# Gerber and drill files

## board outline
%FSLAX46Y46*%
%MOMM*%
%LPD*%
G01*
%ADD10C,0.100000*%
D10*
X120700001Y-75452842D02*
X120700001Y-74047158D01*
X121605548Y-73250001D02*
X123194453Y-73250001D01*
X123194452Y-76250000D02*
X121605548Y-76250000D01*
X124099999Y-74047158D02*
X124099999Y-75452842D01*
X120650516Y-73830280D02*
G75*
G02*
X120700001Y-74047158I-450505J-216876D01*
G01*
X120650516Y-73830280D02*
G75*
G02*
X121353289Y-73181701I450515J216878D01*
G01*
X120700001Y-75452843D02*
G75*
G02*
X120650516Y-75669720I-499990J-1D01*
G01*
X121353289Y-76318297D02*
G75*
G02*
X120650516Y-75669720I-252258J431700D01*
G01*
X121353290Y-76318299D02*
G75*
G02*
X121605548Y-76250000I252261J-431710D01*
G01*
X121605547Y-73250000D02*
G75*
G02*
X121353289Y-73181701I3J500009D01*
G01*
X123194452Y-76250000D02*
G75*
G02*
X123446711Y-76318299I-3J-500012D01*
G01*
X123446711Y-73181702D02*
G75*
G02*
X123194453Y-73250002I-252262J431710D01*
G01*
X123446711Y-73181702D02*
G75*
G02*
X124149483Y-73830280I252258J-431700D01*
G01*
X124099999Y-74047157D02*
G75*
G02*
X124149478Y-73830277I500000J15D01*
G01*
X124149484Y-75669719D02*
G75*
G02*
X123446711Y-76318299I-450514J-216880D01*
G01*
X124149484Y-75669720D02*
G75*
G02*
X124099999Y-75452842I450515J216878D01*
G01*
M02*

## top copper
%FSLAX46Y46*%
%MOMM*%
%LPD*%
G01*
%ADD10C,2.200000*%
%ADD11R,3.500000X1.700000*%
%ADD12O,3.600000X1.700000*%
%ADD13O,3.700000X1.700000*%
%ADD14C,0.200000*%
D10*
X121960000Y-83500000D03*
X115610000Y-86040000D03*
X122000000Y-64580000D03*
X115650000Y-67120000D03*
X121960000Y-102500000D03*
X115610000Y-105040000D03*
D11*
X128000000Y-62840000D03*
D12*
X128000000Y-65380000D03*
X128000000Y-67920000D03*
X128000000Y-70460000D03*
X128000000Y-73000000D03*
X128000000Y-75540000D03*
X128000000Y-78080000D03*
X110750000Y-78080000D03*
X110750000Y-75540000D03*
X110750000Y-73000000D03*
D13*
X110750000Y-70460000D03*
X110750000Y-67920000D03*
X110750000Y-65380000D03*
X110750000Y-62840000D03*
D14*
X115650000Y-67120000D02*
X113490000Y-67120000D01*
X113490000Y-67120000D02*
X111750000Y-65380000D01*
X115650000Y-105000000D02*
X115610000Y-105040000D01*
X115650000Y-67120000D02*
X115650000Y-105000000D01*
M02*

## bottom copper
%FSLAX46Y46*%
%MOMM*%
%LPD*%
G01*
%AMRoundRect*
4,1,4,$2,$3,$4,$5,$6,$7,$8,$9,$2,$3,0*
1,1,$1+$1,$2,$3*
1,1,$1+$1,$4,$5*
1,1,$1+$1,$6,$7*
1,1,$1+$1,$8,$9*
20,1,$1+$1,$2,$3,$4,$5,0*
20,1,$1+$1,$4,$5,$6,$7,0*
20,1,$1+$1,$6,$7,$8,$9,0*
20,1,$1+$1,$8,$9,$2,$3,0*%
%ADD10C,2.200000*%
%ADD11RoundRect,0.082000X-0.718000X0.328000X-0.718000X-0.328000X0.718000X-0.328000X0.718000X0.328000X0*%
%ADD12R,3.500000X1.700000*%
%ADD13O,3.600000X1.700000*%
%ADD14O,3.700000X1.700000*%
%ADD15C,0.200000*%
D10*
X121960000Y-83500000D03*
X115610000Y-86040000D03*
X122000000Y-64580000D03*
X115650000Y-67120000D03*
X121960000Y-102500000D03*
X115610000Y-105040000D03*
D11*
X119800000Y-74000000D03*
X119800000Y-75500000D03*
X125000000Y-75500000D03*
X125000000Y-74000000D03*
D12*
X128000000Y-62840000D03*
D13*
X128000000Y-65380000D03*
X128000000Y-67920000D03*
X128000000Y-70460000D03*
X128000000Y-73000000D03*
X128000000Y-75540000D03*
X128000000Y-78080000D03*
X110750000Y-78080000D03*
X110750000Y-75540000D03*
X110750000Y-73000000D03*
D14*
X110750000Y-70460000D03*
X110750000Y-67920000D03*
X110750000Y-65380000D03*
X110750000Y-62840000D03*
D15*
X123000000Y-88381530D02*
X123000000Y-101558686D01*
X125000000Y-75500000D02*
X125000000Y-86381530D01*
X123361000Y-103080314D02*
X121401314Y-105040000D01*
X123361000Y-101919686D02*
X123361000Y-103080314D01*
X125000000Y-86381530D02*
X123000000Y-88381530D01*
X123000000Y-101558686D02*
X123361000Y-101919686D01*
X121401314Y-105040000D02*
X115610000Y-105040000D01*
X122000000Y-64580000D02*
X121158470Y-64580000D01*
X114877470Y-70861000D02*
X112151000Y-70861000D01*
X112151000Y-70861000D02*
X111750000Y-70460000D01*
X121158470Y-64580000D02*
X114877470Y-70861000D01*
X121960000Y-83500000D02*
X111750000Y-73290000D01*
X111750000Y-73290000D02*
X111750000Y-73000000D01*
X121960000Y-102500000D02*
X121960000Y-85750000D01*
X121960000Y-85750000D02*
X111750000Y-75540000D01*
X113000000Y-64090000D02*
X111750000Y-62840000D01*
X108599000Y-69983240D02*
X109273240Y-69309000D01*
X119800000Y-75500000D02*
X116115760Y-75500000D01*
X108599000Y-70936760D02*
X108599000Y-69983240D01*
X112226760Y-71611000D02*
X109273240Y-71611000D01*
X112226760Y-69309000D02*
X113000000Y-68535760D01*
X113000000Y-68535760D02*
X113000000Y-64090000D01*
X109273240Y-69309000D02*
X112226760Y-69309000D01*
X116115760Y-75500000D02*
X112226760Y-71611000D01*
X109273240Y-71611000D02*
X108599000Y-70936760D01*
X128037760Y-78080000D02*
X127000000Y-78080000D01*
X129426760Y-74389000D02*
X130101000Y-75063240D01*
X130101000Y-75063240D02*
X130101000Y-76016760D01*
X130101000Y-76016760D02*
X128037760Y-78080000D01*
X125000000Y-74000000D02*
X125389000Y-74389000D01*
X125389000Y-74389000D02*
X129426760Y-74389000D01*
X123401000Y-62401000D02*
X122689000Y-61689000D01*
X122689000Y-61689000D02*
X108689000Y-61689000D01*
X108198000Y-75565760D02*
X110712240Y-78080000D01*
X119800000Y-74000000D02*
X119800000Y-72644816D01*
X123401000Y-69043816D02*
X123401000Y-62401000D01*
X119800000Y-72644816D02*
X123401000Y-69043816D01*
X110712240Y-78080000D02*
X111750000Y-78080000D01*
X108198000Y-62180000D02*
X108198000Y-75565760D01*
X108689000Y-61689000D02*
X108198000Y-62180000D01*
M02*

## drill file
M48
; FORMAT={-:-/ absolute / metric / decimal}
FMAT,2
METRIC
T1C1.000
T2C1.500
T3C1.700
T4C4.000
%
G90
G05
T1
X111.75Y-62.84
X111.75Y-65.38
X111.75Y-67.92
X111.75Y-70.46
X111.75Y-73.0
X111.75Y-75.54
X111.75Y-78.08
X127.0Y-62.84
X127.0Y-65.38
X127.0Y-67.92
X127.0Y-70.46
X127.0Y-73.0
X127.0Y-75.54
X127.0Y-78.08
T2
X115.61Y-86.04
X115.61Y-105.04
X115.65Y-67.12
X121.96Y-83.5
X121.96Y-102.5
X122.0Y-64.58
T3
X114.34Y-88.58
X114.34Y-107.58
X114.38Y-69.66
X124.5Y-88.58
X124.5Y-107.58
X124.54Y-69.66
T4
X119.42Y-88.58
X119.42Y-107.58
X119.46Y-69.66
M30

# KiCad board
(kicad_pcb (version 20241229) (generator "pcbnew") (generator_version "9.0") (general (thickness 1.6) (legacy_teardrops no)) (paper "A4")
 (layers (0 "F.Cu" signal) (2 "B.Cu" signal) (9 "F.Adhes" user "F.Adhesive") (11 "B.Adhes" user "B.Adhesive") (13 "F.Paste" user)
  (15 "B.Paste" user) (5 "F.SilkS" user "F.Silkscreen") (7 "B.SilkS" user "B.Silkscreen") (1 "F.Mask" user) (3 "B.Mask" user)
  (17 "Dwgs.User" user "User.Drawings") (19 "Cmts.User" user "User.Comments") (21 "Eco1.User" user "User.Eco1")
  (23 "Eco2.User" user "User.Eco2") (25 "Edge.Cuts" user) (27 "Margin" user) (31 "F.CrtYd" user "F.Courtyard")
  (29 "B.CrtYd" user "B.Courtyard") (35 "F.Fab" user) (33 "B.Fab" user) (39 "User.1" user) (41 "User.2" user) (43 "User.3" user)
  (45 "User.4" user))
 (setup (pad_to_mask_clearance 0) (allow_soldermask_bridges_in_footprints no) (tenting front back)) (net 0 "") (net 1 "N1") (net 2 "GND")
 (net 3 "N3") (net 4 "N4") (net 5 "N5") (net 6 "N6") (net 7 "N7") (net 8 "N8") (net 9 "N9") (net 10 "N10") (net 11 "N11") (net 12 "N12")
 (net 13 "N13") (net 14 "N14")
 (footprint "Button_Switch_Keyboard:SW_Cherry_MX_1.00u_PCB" (layer "F.Cu") (at 121.96 83.5)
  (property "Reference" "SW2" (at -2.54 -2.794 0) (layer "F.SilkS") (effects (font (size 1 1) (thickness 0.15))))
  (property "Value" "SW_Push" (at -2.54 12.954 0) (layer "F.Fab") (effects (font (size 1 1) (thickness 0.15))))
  (pad "" np_thru_hole circle (at -7.62 5.08) (size 1.7 1.7) (drill 1.7) (layers "*.Cu" "*.Mask"))
  (pad "" np_thru_hole circle (at -2.54 5.08) (size 4 4) (drill 4) (layers "*.Cu" "*.Mask"))
  (pad "" np_thru_hole circle (at 2.54 5.08) (size 1.7 1.7) (drill 1.7) (layers "*.Cu" "*.Mask"))
  (pad "1" thru_hole circle (at 0 0) (size 2.2 2.2) (drill 1.5) (layers "*.Cu" "*.Mask") (remove_unused_layers no) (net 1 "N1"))
  (pad "2" thru_hole circle (at -6.35 2.54) (size 2.2 2.2) (drill 1.5) (layers "*.Cu" "*.Mask") (remove_unused_layers no) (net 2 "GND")))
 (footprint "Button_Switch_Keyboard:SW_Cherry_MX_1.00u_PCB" (layer "F.Cu") (at 122 64.58)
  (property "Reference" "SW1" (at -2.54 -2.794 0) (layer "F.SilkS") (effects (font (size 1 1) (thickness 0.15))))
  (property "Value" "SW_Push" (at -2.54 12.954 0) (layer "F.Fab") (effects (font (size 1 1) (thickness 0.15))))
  (pad "" np_thru_hole circle (at -7.62 5.08) (size 1.7 1.7) (drill 1.7) (layers "*.Cu" "*.Mask"))
  (pad "" np_thru_hole circle (at -2.54 5.08) (size 4 4) (drill 4) (layers "*.Cu" "*.Mask"))
  (pad "" np_thru_hole circle (at 2.54 5.08) (size 1.7 1.7) (drill 1.7) (layers "*.Cu" "*.Mask"))
  (pad "1" thru_hole circle (at 0 0) (size 2.2 2.2) (drill 1.5) (layers "*.Cu" "*.Mask") (remove_unused_layers no) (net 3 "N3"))
  (pad "2" thru_hole circle (at -6.35 2.54) (size 2.2 2.2) (drill 1.5) (layers "*.Cu" "*.Mask") (remove_unused_layers no) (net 2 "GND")))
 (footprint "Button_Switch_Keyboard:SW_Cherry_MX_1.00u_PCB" (layer "F.Cu") (at 121.96 102.5)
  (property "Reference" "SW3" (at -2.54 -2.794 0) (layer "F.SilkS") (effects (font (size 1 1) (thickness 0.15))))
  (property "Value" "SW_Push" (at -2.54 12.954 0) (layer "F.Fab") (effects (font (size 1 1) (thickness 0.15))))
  (pad "" np_thru_hole circle (at -7.62 5.08) (size 1.7 1.7) (drill 1.7) (layers "*.Cu" "*.Mask"))
  (pad "" np_thru_hole circle (at -2.54 5.08) (size 4 4) (drill 4) (layers "*.Cu" "*.Mask"))
  (pad "" np_thru_hole circle (at 2.54 5.08) (size 1.7 1.7) (drill 1.7) (layers "*.Cu" "*.Mask"))
  (pad "1" thru_hole circle (at 0 0) (size 2.2 2.2) (drill 1.5) (layers "*.Cu" "*.Mask") (remove_unused_layers no) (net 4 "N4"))
  (pad "2" thru_hole circle (at -6.35 2.54) (size 2.2 2.2) (drill 1.5) (layers "*.Cu" "*.Mask") (remove_unused_layers no) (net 2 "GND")))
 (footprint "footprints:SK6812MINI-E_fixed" (layer "F.Cu") (at 122.399999 74.852842)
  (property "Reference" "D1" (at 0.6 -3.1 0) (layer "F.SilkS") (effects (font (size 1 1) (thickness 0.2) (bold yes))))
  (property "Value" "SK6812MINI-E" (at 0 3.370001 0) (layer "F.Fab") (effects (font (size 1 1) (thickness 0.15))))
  (fp_line (start -1.699998 0.6) (end -1.699998 -0.805684) (stroke (width 0.1) (type solid)) (layer "Edge.Cuts"))
  (fp_line (start -0.794451 -1.602841) (end 0.794454 -1.602841) (stroke (width 0.1) (type solid)) (layer "Edge.Cuts"))
  (fp_line (start 0.794453 1.397158) (end -0.794451 1.397158) (stroke (width 0.1) (type solid)) (layer "Edge.Cuts"))
  (fp_line (start 1.7 -0.805684) (end 1.7 0.6) (stroke (width 0.1) (type solid)) (layer "Edge.Cuts"))
  (fp_arc (start -1.749483 -1.022562) (mid -1.712526 -0.91691) (end -1.699998 -0.805684) (stroke (width 0.1) (type solid))
   (layer "Edge.Cuts"))
  (fp_arc (start -1.749483 -1.022562) (mid -1.63807 -1.606877) (end -1.04671 -1.671141) (stroke (width 0.1) (type solid))
   (layer "Edge.Cuts"))
  (fp_arc (start -1.699998 0.600001) (mid -1.712526 0.711226) (end -1.749483 0.816878) (stroke (width 0.1) (type solid)) (layer "Edge.Cuts"))
  (fp_arc (start -1.04671 1.465455) (mid -1.638069 1.401192) (end -1.749483 0.816878) (stroke (width 0.1) (type solid)) (layer "Edge.Cuts"))
  (fp_arc (start -1.046709 1.465457) (mid -0.925121 1.414535) (end -0.794451 1.397158) (stroke (width 0.1) (type solid)) (layer "Edge.Cuts"))
  (fp_arc (start -0.794452 -1.602842) (mid -0.925122 -1.620219) (end -1.04671 -1.671141) (stroke (width 0.1) (type solid))
   (layer "Edge.Cuts"))
  (fp_arc (start 0.794453 1.397158) (mid 0.925124 1.414535) (end 1.046712 1.465457) (stroke (width 0.1) (type solid)) (layer "Edge.Cuts"))
  (fp_arc (start 1.046712 -1.67114) (mid 0.925124 -1.620218) (end 0.794454 -1.602841) (stroke (width 0.1) (type solid)) (layer "Edge.Cuts"))
  (fp_arc (start 1.046712 -1.67114) (mid 1.638072 -1.606876) (end 1.749485 -1.022562) (stroke (width 0.1) (type solid)) (layer "Edge.Cuts"))
  (fp_arc (start 1.7 -0.805685) (mid 1.712528 -0.91691) (end 1.749485 -1.022562) (stroke (width 0.1) (type solid)) (layer "Edge.Cuts"))
  (fp_arc (start 1.749485 0.816877) (mid 1.638073 1.401193) (end 1.046712 1.465457) (stroke (width 0.1) (type solid)) (layer "Edge.Cuts"))
  (fp_arc (start 1.749485 0.816878) (mid 1.712528 0.711226) (end 1.7 0.6) (stroke (width 0.1) (type solid)) (layer "Edge.Cuts"))
  (pad "1" smd roundrect (at -2.599999 -0.852842 270) (size 0.82 1.6) (layers "B.Cu" "B.Mask" "B.Paste") (roundrect_rratio 0.1) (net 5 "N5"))
  (pad "2" smd roundrect (at -2.599999 0.647158 270) (size 0.82 1.6) (layers "B.Cu" "B.Mask" "B.Paste") (roundrect_rratio 0.1) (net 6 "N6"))
  (pad "3" smd roundrect (at 2.600001 0.647158 270) (size 0.82 1.6) (layers "B.Cu" "B.Mask" "B.Paste") (roundrect_rratio 0.1) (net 2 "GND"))
  (pad "4" smd roundrect (at 2.600001 -0.852842 270) (size 0.82 1.6) (layers "B.Cu" "B.Mask" "B.Paste") (roundrect_rratio 0.1) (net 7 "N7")))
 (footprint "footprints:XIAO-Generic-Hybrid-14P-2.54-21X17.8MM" (layer "B.Cu") (at 119.375 70.46 180)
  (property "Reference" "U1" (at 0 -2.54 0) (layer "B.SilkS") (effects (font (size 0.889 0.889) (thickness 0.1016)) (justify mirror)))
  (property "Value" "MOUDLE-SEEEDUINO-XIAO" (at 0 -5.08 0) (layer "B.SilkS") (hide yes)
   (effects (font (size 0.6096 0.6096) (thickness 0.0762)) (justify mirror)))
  (pad "1" thru_hole rect (at -7.625 7.62 180) (size 3.5 1.7) (drill 1 (offset -1 0)) (layers "*.Cu" "*.Mask") (remove_unused_layers no)
   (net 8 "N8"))
  (pad "2" thru_hole oval (at -7.625 5.08 180) (size 3.6 1.7) (drill 1 (offset -1 0)) (layers "*.Cu" "*.Mask") (remove_unused_layers no)
   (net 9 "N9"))
  (pad "3" thru_hole oval (at -7.625 2.54 180) (size 3.6 1.7) (drill 1 (offset -1 0)) (layers "*.Cu" "*.Mask") (remove_unused_layers no)
   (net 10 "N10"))
  (pad "4" thru_hole oval (at -7.625 0 180) (size 3.6 1.7) (drill 1 (offset -1 0)) (layers "*.Cu" "*.Mask") (remove_unused_layers no)
   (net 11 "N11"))
  (pad "5" thru_hole oval (at -7.625 -2.54 180) (size 3.6 1.7) (drill 1 (offset -1 0)) (layers "*.Cu" "*.Mask") (remove_unused_layers no)
   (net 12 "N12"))
  (pad "6" thru_hole oval (at -7.625 -5.08) (size 3.6 1.7) (drill 1 (offset 1 0)) (layers "*.Cu" "*.Mask") (remove_unused_layers no)
   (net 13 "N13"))
  (pad "7" thru_hole oval (at -7.625 -7.62 180) (size 3.6 1.7) (drill 1 (offset -1 0)) (layers "*.Cu" "*.Mask") (remove_unused_layers no)
   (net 7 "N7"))
  (pad "8" thru_hole oval (at 7.625 -7.62 180) (size 3.6 1.7) (drill 1 (offset 1 0)) (layers "*.Cu" "*.Mask") (remove_unused_layers no)
   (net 5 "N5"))
  (pad "9" thru_hole oval (at 7.625 -5.08 180) (size 3.6 1.7) (drill 1 (offset 1 0)) (layers "*.Cu" "*.Mask") (remove_unused_layers no)
   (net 4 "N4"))
  (pad "10" thru_hole oval (at 7.625 -2.54 180) (size 3.6 1.7) (drill 1 (offset 1 0)) (layers "*.Cu" "*.Mask") (remove_unused_layers no)
   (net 1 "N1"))
  (pad "11" thru_hole oval (at 7.625 0 180) (size 3.7 1.7) (drill 1 (offset 1 0)) (layers "*.Cu" "*.Mask") (remove_unused_layers no)
   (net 3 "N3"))
  (pad "12" thru_hole oval (at 7.625 2.54 180) (size 3.7 1.7) (drill 1 (offset 1 0)) (layers "*.Cu" "*.Mask") (remove_unused_layers no)
   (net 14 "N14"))
  (pad "13" thru_hole oval (at 7.625 5.08 180) (size 3.7 1.7) (drill 1 (offset 1 0)) (layers "*.Cu" "*.Mask") (remove_unused_layers no)
   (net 2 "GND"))
  (pad "14" thru_hole oval (at 7.625 7.62 180) (size 3.7 1.7) (drill 1 (offset 1 0)) (layers "*.Cu" "*.Mask") (remove_unused_layers no)
   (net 6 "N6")))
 (segment (start 115.65 67.12) (end 113.49 67.12) (width 0.2) (layer "F.Cu") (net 2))
 (segment (start 113.49 67.12) (end 111.75 65.38) (width 0.2) (layer "F.Cu") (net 2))
 (segment (start 115.65 105) (end 115.61 105.04) (width 0.2) (layer "F.Cu") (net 2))
 (segment (start 115.65 67.12) (end 115.65 105) (width 0.2) (layer "F.Cu") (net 2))
 (segment (start 123 88.38153) (end 123 101.558686) (width 0.2) (layer "B.Cu") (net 2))
 (segment (start 125 75.5) (end 125 86.38153) (width 0.2) (layer "B.Cu") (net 2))
 (segment (start 123.361 103.080314) (end 121.401314 105.04) (width 0.2) (layer "B.Cu") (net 2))
 (segment (start 123.361 101.919686) (end 123.361 103.080314) (width 0.2) (layer "B.Cu") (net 2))
 (segment (start 125 86.38153) (end 123 88.38153) (width 0.2) (layer "B.Cu") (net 2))
 (segment (start 123 101.558686) (end 123.361 101.919686) (width 0.2) (layer "B.Cu") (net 2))
 (segment (start 121.401314 105.04) (end 115.61 105.04) (width 0.2) (layer "B.Cu") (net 2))
 (segment (start 122 64.58) (end 121.15847 64.58) (width 0.2) (layer "B.Cu") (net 3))
 (segment (start 114.87747 70.861) (end 112.151 70.861) (width 0.2) (layer "B.Cu") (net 3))
 (segment (start 112.151 70.861) (end 111.75 70.46) (width 0.2) (layer "B.Cu") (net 3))
 (segment (start 121.15847 64.58) (end 114.87747 70.861) (width 0.2) (layer "B.Cu") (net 3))
 (segment (start 121.96 83.5) (end 111.75 73.29) (width 0.2) (layer "B.Cu") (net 1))
 (segment (start 111.75 73.29) (end 111.75 73) (width 0.2) (layer "B.Cu") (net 1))
 (segment (start 121.96 102.5) (end 121.96 85.75) (width 0.2) (layer "B.Cu") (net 4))
 (segment (start 121.96 85.75) (end 111.75 75.54) (width 0.2) (layer "B.Cu") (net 4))
 (segment (start 113 64.09) (end 111.75 62.84) (width 0.2) (layer "B.Cu") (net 6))
 (segment (start 108.599 69.98324) (end 109.27324 69.309) (width 0.2) (layer "B.Cu") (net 6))
 (segment (start 119.8 75.5) (end 116.11576 75.5) (width 0.2) (layer "B.Cu") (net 6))
 (segment (start 108.599 70.93676) (end 108.599 69.98324) (width 0.2) (layer "B.Cu") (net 6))
 (segment (start 112.22676 71.611) (end 109.27324 71.611) (width 0.2) (layer "B.Cu") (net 6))
 (segment (start 112.22676 69.309) (end 113 68.53576) (width 0.2) (layer "B.Cu") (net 6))
 (segment (start 113 68.53576) (end 113 64.09) (width 0.2) (layer "B.Cu") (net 6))
 (segment (start 109.27324 69.309) (end 112.22676 69.309) (width 0.2) (layer "B.Cu") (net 6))
 (segment (start 116.11576 75.5) (end 112.22676 71.611) (width 0.2) (layer "B.Cu") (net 6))
 (segment (start 109.27324 71.611) (end 108.599 70.93676) (width 0.2) (layer "B.Cu") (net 6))
 (segment (start 128.03776 78.08) (end 127 78.08) (width 0.2) (layer "B.Cu") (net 7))
 (segment (start 129.42676 74.389) (end 130.101 75.06324) (width 0.2) (layer "B.Cu") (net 7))
 (segment (start 130.101 75.06324) (end 130.101 76.01676) (width 0.2) (layer "B.Cu") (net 7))
 (segment (start 130.101 76.01676) (end 128.03776 78.08) (width 0.2) (layer "B.Cu") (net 7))
 (segment (start 125 74) (end 125.389 74.389) (width 0.2) (layer "B.Cu") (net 7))
 (segment (start 125.389 74.389) (end 129.42676 74.389) (width 0.2) (layer "B.Cu") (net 7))
 (segment (start 123.401 62.401) (end 122.689 61.689) (width 0.2) (layer "B.Cu") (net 5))
 (segment (start 122.689 61.689) (end 108.689 61.689) (width 0.2) (layer "B.Cu") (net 5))
 (segment (start 108.198 75.56576) (end 110.71224 78.08) (width 0.2) (layer "B.Cu") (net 5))
 (segment (start 119.8 74) (end 119.8 72.644816) (width 0.2) (layer "B.Cu") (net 5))
 (segment (start 123.401 69.043816) (end 123.401 62.401) (width 0.2) (layer "B.Cu") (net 5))
 (segment (start 119.8 72.644816) (end 123.401 69.043816) (width 0.2) (layer "B.Cu") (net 5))
 (segment (start 110.71224 78.08) (end 111.75 78.08) (width 0.2) (layer "B.Cu") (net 5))
 (segment (start 108.198 62.18) (end 108.198 75.56576) (width 0.2) (layer "B.Cu") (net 5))
 (segment (start 108.689 61.689) (end 108.198 62.18) (width 0.2) (layer "B.Cu") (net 5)))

